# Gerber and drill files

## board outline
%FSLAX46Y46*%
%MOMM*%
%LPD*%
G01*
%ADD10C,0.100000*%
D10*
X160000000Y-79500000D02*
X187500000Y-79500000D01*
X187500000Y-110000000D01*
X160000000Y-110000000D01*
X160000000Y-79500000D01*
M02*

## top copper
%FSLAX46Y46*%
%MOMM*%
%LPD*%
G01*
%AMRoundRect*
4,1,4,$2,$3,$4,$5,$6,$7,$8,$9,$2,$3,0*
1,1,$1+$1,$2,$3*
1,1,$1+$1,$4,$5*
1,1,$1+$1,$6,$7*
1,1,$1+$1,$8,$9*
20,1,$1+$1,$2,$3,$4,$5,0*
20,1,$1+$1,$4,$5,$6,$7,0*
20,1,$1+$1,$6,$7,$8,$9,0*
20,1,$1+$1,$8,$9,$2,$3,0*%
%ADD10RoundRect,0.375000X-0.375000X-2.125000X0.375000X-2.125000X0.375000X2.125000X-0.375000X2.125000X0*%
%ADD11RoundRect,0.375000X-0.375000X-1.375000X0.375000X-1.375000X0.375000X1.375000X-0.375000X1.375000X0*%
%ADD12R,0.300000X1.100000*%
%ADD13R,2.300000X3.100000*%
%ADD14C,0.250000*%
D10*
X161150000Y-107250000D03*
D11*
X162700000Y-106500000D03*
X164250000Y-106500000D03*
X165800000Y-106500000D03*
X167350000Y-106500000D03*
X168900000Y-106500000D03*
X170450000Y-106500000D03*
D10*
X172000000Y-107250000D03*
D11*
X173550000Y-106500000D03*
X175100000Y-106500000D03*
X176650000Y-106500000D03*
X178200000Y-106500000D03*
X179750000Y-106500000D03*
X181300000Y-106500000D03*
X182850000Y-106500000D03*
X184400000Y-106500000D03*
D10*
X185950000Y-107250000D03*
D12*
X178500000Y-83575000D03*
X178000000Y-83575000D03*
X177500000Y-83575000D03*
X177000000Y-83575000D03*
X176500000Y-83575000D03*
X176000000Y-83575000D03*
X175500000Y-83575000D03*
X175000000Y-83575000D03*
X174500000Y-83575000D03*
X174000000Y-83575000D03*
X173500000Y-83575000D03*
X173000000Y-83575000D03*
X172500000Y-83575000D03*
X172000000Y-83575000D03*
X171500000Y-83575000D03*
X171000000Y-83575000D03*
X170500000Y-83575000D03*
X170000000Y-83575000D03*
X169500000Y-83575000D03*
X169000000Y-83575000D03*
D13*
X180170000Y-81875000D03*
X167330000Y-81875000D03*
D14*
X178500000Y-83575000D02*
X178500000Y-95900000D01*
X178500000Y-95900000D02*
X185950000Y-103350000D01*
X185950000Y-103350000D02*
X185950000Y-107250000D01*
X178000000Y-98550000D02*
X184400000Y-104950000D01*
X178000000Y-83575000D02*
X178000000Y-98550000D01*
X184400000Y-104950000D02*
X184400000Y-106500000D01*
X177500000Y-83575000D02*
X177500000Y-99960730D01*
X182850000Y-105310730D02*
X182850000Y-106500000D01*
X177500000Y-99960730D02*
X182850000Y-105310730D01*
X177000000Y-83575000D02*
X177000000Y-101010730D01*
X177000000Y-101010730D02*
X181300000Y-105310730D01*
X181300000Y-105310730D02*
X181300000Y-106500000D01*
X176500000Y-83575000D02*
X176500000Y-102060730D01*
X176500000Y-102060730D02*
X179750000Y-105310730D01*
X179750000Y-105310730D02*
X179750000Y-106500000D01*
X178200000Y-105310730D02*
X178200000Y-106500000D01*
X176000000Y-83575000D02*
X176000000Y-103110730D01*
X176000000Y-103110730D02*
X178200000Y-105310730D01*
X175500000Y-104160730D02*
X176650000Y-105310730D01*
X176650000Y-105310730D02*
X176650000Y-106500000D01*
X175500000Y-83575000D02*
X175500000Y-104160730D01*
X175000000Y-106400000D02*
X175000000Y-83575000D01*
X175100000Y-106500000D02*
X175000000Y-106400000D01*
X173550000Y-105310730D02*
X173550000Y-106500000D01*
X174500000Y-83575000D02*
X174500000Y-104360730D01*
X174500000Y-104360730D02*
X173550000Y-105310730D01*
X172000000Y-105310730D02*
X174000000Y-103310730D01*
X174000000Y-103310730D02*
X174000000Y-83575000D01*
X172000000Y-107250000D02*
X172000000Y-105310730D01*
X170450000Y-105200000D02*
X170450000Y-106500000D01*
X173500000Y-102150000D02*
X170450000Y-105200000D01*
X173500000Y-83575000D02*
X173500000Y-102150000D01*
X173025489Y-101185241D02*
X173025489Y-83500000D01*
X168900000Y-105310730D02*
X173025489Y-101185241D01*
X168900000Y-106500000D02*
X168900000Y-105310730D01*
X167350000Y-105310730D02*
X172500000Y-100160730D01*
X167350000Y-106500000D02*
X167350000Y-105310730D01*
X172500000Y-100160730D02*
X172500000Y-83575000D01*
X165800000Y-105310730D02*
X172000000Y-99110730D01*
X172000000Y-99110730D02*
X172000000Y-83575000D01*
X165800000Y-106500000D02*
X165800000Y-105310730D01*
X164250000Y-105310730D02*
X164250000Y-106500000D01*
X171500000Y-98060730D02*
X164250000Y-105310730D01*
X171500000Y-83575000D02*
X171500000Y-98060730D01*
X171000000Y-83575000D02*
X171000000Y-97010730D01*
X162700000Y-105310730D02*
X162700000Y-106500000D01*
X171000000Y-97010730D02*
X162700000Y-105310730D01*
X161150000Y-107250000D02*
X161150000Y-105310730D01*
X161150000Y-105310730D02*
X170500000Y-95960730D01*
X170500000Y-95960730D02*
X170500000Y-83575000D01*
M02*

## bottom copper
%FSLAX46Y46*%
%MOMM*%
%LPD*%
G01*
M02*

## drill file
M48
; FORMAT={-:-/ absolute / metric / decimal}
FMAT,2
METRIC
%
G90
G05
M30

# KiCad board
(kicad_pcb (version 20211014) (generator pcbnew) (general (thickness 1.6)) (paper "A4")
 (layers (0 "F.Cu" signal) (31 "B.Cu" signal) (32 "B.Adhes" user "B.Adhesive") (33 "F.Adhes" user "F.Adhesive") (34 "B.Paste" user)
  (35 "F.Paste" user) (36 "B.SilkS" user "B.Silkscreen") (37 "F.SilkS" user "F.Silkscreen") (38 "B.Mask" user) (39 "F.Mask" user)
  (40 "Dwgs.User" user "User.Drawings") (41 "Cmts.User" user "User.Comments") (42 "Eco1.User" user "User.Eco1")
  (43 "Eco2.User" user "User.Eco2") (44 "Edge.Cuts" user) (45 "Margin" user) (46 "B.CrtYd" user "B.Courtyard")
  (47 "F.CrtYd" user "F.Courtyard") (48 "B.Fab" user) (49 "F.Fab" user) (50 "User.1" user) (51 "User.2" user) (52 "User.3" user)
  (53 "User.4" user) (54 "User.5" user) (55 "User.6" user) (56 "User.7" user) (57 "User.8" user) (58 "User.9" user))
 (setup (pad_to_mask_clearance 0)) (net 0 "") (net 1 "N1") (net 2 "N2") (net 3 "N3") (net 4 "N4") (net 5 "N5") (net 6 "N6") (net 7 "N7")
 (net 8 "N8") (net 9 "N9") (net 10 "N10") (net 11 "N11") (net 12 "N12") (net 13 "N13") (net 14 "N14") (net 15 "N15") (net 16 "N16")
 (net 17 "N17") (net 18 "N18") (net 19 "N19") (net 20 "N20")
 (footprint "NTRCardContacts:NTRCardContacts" (layer "F.Cu") (at 167.4 112.75)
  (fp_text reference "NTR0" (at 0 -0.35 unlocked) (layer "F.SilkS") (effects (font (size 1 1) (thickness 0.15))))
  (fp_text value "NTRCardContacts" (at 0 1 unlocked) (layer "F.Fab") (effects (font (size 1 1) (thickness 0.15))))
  (pad "1" smd roundrect (at -6.25 -5.5) (size 1.5 5) (layers "F.Cu" "F.Paste" "F.Mask") (roundrect_rratio 0.25) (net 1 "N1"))
  (pad "2" smd roundrect (at -4.7 -6.25) (size 1.5 3.5) (layers "F.Cu" "F.Paste" "F.Mask") (roundrect_rratio 0.25) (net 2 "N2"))
  (pad "3" smd roundrect (at -3.15 -6.25) (size 1.5 3.5) (layers "F.Cu" "F.Paste" "F.Mask") (roundrect_rratio 0.25) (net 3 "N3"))
  (pad "4" smd roundrect (at -1.6 -6.25) (size 1.5 3.5) (layers "F.Cu" "F.Paste" "F.Mask") (roundrect_rratio 0.25) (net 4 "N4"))
  (pad "5" smd roundrect (at -0.05 -6.25) (size 1.5 3.5) (layers "F.Cu" "F.Paste" "F.Mask") (roundrect_rratio 0.25) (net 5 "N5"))
  (pad "6" smd roundrect (at 1.5 -6.25) (size 1.5 3.5) (layers "F.Cu" "F.Paste" "F.Mask") (roundrect_rratio 0.25) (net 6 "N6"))
  (pad "7" smd roundrect (at 3.05 -6.25) (size 1.5 3.5) (layers "F.Cu" "F.Paste" "F.Mask") (roundrect_rratio 0.25) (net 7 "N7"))
  (pad "8" smd roundrect (at 4.6 -5.5) (size 1.5 5) (layers "F.Cu" "F.Paste" "F.Mask") (roundrect_rratio 0.25) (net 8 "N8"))
  (pad "9" smd roundrect (at 6.15 -6.25) (size 1.5 3.5) (layers "F.Cu" "F.Paste" "F.Mask") (roundrect_rratio 0.25) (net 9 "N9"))
  (pad "10" smd roundrect (at 7.7 -6.25) (size 1.5 3.5) (layers "F.Cu" "F.Paste" "F.Mask") (roundrect_rratio 0.25) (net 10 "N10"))
  (pad "11" smd roundrect (at 9.25 -6.25) (size 1.5 3.5) (layers "F.Cu" "F.Paste" "F.Mask") (roundrect_rratio 0.25) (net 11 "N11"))
  (pad "12" smd roundrect (at 10.8 -6.25) (size 1.5 3.5) (layers "F.Cu" "F.Paste" "F.Mask") (roundrect_rratio 0.25) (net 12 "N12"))
  (pad "13" smd roundrect (at 12.35 -6.25) (size 1.5 3.5) (layers "F.Cu" "F.Paste" "F.Mask") (roundrect_rratio 0.25) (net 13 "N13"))
  (pad "14" smd roundrect (at 13.9 -6.25) (size 1.5 3.5) (layers "F.Cu" "F.Paste" "F.Mask") (roundrect_rratio 0.25) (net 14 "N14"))
  (pad "15" smd roundrect (at 15.45 -6.25) (size 1.5 3.5) (layers "F.Cu" "F.Paste" "F.Mask") (roundrect_rratio 0.25) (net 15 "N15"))
  (pad "16" smd roundrect (at 17 -6.25) (size 1.5 3.5) (layers "F.Cu" "F.Paste" "F.Mask") (roundrect_rratio 0.25) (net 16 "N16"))
  (pad "17" smd roundrect (at 18.55 -5.5) (size 1.5 5) (layers "F.Cu" "F.Paste" "F.Mask") (roundrect_rratio 0.25) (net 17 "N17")))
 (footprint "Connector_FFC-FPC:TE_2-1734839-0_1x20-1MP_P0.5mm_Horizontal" (layer "F.Cu") (at 173.75 82.225 180)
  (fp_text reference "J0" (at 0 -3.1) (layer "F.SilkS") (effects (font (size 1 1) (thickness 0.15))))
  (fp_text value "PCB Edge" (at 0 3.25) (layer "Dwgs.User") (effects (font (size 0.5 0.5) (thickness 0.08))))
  (pad "1" smd rect (at -4.75 -1.35 180) (size 0.3 1.1) (layers "F.Cu" "F.Paste" "F.Mask") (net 17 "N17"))
  (pad "2" smd rect (at -4.25 -1.35 180) (size 0.3 1.1) (layers "F.Cu" "F.Paste" "F.Mask") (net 16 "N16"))
  (pad "3" smd rect (at -3.75 -1.35 180) (size 0.3 1.1) (layers "F.Cu" "F.Paste" "F.Mask") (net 15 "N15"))
  (pad "4" smd rect (at -3.25 -1.35 180) (size 0.3 1.1) (layers "F.Cu" "F.Paste" "F.Mask") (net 14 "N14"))
  (pad "5" smd rect (at -2.75 -1.35 180) (size 0.3 1.1) (layers "F.Cu" "F.Paste" "F.Mask") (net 13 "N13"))
  (pad "6" smd rect (at -2.25 -1.35 180) (size 0.3 1.1) (layers "F.Cu" "F.Paste" "F.Mask") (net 12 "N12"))
  (pad "7" smd rect (at -1.75 -1.35 180) (size 0.3 1.1) (layers "F.Cu" "F.Paste" "F.Mask") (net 11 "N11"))
  (pad "8" smd rect (at -1.25 -1.35 180) (size 0.3 1.1) (layers "F.Cu" "F.Paste" "F.Mask") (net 10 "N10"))
  (pad "9" smd rect (at -0.75 -1.35 180) (size 0.3 1.1) (layers "F.Cu" "F.Paste" "F.Mask") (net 9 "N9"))
  (pad "10" smd rect (at -0.25 -1.35 180) (size 0.3 1.1) (layers "F.Cu" "F.Paste" "F.Mask") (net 8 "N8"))
  (pad "11" smd rect (at 0.25 -1.35 180) (size 0.3 1.1) (layers "F.Cu" "F.Paste" "F.Mask") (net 7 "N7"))
  (pad "12" smd rect (at 0.75 -1.35 180) (size 0.3 1.1) (layers "F.Cu" "F.Paste" "F.Mask") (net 6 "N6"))
  (pad "13" smd rect (at 1.25 -1.35 180) (size 0.3 1.1) (layers "F.Cu" "F.Paste" "F.Mask") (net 5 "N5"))
  (pad "14" smd rect (at 1.75 -1.35 180) (size 0.3 1.1) (layers "F.Cu" "F.Paste" "F.Mask") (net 4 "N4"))
  (pad "15" smd rect (at 2.25 -1.35 180) (size 0.3 1.1) (layers "F.Cu" "F.Paste" "F.Mask") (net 3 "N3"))
  (pad "16" smd rect (at 2.75 -1.35 180) (size 0.3 1.1) (layers "F.Cu" "F.Paste" "F.Mask") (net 2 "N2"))
  (pad "17" smd rect (at 3.25 -1.35 180) (size 0.3 1.1) (layers "F.Cu" "F.Paste" "F.Mask") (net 1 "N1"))
  (pad "18" smd rect (at 3.75 -1.35 180) (size 0.3 1.1) (layers "F.Cu" "F.Paste" "F.Mask") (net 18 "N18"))
  (pad "19" smd rect (at 4.25 -1.35 180) (size 0.3 1.1) (layers "F.Cu" "F.Paste" "F.Mask") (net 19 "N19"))
  (pad "20" smd rect (at 4.75 -1.35 180) (size 0.3 1.1) (layers "F.Cu" "F.Paste" "F.Mask") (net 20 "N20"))
  (pad "MP" smd rect (at -6.42 0.35 180) (size 2.3 3.1) (layers "F.Cu" "F.Paste" "F.Mask"))
  (pad "MP" smd rect (at 6.42 0.35 180) (size 2.3 3.1) (layers "F.Cu" "F.Paste" "F.Mask")))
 (gr_rect locked (start 160 79.5) (end 187.5 110) (layer "Edge.Cuts") (width 0.1) (fill none))
 (segment (start 178.5 83.575) (end 178.5 95.9) (width 0.25) (layer "F.Cu") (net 17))
 (segment (start 178.5 95.9) (end 185.95 103.35) (width 0.25) (layer "F.Cu") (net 17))
 (segment (start 185.95 103.35) (end 185.95 107.25) (width 0.25) (layer "F.Cu") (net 17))
 (segment (start 178 98.55) (end 184.4 104.95) (width 0.25) (layer "F.Cu") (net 16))
 (segment (start 178 83.575) (end 178 98.55) (width 0.25) (layer "F.Cu") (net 16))
 (segment (start 184.4 104.95) (end 184.4 106.5) (width 0.25) (layer "F.Cu") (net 16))
 (segment (start 177.5 83.575) (end 177.5 99.96073) (width 0.25) (layer "F.Cu") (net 15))
 (segment (start 182.85 105.31073) (end 182.85 106.5) (width 0.25) (layer "F.Cu") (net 15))
 (segment (start 177.5 99.96073) (end 182.85 105.31073) (width 0.25) (layer "F.Cu") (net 15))
 (segment (start 177 83.575) (end 177 101.01073) (width 0.25) (layer "F.Cu") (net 14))
 (segment (start 177 101.01073) (end 181.3 105.31073) (width 0.25) (layer "F.Cu") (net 14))
 (segment (start 181.3 105.31073) (end 181.3 106.5) (width 0.25) (layer "F.Cu") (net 14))
 (segment (start 176.5 83.575) (end 176.5 102.06073) (width 0.25) (layer "F.Cu") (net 13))
 (segment (start 176.5 102.06073) (end 179.75 105.31073) (width 0.25) (layer "F.Cu") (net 13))
 (segment (start 179.75 105.31073) (end 179.75 106.5) (width 0.25) (layer "F.Cu") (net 13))
 (segment (start 178.2 105.31073) (end 178.2 106.5) (width 0.25) (layer "F.Cu") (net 12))
 (segment (start 176 83.575) (end 176 103.11073) (width 0.25) (layer "F.Cu") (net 12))
 (segment (start 176 103.11073) (end 178.2 105.31073) (width 0.25) (layer "F.Cu") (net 12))
 (segment (start 175.5 104.16073) (end 176.65 105.31073) (width 0.25) (layer "F.Cu") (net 11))
 (segment (start 176.65 105.31073) (end 176.65 106.5) (width 0.25) (layer "F.Cu") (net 11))
 (segment (start 175.5 83.575) (end 175.5 104.16073) (width 0.25) (layer "F.Cu") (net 11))
 (segment (start 175 106.4) (end 175 83.575) (width 0.25) (layer "F.Cu") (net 10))
 (segment (start 175.1 106.5) (end 175 106.4) (width 0.25) (layer "F.Cu") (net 10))
 (segment (start 173.55 105.31073) (end 173.55 106.5) (width 0.25) (layer "F.Cu") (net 9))
 (segment (start 174.5 83.575) (end 174.5 104.36073) (width 0.25) (layer "F.Cu") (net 9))
 (segment (start 174.5 104.36073) (end 173.55 105.31073) (width 0.25) (layer "F.Cu") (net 9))
 (segment (start 172 105.31073) (end 174 103.31073) (width 0.25) (layer "F.Cu") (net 8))
 (segment (start 174 103.31073) (end 174 83.575) (width 0.25) (layer "F.Cu") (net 8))
 (segment (start 172 107.25) (end 172 105.31073) (width 0.25) (layer "F.Cu") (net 8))
 (segment (start 170.45 105.2) (end 170.45 106.5) (width 0.25) (layer "F.Cu") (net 7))
 (segment (start 173.5 102.15) (end 170.45 105.2) (width 0.25) (layer "F.Cu") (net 7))
 (segment (start 173.5 83.575) (end 173.5 102.15) (width 0.25) (layer "F.Cu") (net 7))
 (segment (start 173.025489 101.185241) (end 173.025489 83.5) (width 0.25) (layer "F.Cu") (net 6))
 (segment (start 168.9 105.31073) (end 173.025489 101.185241) (width 0.25) (layer "F.Cu") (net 6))
 (segment (start 168.9 106.5) (end 168.9 105.31073) (width 0.25) (layer "F.Cu") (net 6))
 (segment (start 167.35 105.31073) (end 172.5 100.16073) (width 0.25) (layer "F.Cu") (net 5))
 (segment (start 167.35 106.5) (end 167.35 105.31073) (width 0.25) (layer "F.Cu") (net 5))
 (segment (start 172.5 100.16073) (end 172.5 83.575) (width 0.25) (layer "F.Cu") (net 5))
 (segment (start 165.8 105.31073) (end 172 99.11073) (width 0.25) (layer "F.Cu") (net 4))
 (segment (start 172 99.11073) (end 172 83.575) (width 0.25) (layer "F.Cu") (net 4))
 (segment (start 165.8 106.5) (end 165.8 105.31073) (width 0.25) (layer "F.Cu") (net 4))
 (segment (start 164.25 105.31073) (end 164.25 106.5) (width 0.25) (layer "F.Cu") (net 3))
 (segment (start 171.5 98.06073) (end 164.25 105.31073) (width 0.25) (layer "F.Cu") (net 3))
 (segment (start 171.5 83.575) (end 171.5 98.06073) (width 0.25) (layer "F.Cu") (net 3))
 (segment (start 171 83.575) (end 171 97.01073) (width 0.25) (layer "F.Cu") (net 2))
 (segment (start 162.7 105.31073) (end 162.7 106.5) (width 0.25) (layer "F.Cu") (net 2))
 (segment (start 171 97.01073) (end 162.7 105.31073) (width 0.25) (layer "F.Cu") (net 2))
 (segment (start 161.15 107.25) (end 161.15 105.31073) (width 0.25) (layer "F.Cu") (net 1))
 (segment (start 161.15 105.31073) (end 170.5 95.96073) (width 0.25) (layer "F.Cu") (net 1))
 (segment (start 170.5 95.96073) (end 170.5 83.575) (width 0.25) (layer "F.Cu") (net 1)))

